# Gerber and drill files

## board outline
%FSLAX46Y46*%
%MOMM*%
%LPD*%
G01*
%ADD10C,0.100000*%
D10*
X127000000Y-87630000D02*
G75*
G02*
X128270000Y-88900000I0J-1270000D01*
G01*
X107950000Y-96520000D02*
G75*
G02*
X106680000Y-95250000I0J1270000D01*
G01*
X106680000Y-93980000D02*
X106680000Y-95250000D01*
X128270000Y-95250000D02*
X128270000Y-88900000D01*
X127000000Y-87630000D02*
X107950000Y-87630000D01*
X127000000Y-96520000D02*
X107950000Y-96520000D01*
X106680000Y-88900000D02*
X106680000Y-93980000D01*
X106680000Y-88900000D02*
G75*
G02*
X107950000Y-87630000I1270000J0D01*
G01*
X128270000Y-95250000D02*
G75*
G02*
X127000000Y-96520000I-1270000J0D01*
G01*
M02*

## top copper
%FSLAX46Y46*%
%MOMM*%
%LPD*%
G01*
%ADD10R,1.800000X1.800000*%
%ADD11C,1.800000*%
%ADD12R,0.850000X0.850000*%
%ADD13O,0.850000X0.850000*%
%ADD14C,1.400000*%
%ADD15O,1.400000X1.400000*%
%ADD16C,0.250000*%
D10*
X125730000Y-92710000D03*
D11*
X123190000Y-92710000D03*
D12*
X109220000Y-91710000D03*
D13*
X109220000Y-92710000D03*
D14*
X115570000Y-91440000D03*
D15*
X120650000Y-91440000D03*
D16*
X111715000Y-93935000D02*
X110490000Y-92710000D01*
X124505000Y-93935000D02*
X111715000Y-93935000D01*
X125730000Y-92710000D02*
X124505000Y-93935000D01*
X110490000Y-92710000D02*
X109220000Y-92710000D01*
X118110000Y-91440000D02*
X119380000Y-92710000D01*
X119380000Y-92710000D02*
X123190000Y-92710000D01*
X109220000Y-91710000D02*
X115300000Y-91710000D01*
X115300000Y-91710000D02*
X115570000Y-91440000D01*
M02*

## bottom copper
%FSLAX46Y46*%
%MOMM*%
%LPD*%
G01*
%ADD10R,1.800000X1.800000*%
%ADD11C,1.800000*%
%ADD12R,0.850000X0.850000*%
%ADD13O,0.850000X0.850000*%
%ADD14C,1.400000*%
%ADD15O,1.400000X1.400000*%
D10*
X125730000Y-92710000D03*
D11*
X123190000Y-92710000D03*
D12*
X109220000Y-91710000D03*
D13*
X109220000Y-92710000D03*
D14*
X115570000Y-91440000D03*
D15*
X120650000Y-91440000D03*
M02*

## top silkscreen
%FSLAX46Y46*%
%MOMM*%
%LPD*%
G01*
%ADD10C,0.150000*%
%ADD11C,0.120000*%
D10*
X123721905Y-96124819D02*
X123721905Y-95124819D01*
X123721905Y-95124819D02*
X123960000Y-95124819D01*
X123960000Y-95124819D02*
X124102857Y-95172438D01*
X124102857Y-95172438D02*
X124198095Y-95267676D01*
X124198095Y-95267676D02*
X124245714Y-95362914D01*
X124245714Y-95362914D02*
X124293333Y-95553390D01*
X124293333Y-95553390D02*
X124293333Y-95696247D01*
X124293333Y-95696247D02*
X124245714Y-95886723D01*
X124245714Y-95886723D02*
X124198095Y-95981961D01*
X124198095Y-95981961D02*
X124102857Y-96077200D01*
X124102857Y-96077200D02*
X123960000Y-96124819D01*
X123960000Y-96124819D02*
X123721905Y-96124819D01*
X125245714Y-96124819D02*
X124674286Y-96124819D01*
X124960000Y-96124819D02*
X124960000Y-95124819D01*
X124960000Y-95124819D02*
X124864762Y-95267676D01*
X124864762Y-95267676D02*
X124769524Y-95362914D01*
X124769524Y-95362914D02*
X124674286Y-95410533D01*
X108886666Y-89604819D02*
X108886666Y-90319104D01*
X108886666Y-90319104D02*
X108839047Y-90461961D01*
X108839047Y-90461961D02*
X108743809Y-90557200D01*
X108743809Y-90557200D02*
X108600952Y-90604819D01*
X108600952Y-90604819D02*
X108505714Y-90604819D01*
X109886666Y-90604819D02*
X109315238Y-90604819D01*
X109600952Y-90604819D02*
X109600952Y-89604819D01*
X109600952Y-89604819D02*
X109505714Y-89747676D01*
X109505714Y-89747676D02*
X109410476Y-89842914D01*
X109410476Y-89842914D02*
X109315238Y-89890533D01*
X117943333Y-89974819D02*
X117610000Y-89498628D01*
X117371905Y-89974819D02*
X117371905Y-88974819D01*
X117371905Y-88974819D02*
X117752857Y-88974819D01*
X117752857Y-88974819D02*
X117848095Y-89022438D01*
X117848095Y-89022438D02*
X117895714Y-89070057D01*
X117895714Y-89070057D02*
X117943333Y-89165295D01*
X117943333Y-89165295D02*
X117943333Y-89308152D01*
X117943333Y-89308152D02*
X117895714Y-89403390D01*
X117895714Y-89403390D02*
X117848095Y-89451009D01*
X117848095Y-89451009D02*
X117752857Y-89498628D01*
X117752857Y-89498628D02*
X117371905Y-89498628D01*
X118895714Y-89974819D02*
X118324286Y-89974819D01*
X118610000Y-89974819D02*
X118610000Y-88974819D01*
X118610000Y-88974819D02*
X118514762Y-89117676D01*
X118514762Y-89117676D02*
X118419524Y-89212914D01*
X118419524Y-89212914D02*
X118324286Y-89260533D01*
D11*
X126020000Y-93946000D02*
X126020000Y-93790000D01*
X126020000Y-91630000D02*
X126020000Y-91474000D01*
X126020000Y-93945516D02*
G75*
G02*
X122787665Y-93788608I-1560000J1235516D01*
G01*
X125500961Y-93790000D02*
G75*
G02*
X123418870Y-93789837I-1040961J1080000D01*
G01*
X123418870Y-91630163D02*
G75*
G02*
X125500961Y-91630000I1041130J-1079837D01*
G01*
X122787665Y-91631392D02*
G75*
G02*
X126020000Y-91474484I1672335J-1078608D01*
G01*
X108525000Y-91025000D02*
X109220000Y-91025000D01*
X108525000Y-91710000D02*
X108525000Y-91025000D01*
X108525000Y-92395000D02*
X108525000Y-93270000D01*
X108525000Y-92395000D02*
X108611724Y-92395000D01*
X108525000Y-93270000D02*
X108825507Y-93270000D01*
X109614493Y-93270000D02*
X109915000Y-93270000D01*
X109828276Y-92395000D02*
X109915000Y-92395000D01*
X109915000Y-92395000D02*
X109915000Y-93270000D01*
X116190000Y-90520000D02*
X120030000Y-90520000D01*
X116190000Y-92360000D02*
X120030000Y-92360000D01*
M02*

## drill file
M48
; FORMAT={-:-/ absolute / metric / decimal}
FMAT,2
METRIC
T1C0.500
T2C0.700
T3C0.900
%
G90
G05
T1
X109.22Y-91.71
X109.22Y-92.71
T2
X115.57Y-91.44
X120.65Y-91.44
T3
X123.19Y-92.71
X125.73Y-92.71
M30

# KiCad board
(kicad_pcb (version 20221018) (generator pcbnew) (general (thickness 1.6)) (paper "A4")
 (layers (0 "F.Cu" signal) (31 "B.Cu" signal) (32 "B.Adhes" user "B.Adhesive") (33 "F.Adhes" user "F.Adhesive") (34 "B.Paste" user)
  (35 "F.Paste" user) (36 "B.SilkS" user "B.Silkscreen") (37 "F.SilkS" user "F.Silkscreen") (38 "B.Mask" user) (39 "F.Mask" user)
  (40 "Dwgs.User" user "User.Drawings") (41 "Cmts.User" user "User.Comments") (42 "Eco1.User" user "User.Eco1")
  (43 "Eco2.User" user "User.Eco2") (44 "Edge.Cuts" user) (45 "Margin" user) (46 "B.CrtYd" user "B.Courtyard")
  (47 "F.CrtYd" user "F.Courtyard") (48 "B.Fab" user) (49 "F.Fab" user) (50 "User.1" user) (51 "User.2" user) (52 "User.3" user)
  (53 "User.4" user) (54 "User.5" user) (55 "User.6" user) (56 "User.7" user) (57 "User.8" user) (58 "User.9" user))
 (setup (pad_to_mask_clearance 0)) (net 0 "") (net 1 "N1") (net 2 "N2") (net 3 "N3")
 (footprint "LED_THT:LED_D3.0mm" (layer "F.Cu") (at 125.73 92.71 180)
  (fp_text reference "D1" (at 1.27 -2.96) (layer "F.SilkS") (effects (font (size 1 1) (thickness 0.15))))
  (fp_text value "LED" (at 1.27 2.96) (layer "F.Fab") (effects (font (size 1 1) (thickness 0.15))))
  (fp_line (start -0.29 -1.236) (end -0.29 -1.08) (stroke (width 0.12) (type solid)) (layer "F.SilkS"))
  (fp_line (start -0.29 1.08) (end -0.29 1.236) (stroke (width 0.12) (type solid)) (layer "F.SilkS"))
  (fp_arc (start -0.29 -1.235516) (mid 1.366487 -1.987659) (end 2.942335 -1.078608) (stroke (width 0.12) (type solid)) (layer "F.SilkS"))
  (fp_arc (start 0.229039 -1.08) (mid 1.270117 -1.5) (end 2.31113 -1.079837) (stroke (width 0.12) (type solid)) (layer "F.SilkS"))
  (fp_arc (start 2.31113 1.079837) (mid 1.270117 1.5) (end 0.229039 1.08) (stroke (width 0.12) (type solid)) (layer "F.SilkS"))
  (fp_arc (start 2.942335 1.078608) (mid 1.366487 1.987659) (end -0.29 1.235516) (stroke (width 0.12) (type solid)) (layer "F.SilkS"))
  (pad "1" thru_hole rect (at 0 0 180) (size 1.8 1.8) (drill 0.9) (layers "*.Cu" "*.Mask") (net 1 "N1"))
  (pad "2" thru_hole circle (at 2.54 0 180) (size 1.8 1.8) (drill 0.9) (layers "*.Cu" "*.Mask") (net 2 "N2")))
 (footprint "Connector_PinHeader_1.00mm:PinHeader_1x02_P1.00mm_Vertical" (layer "F.Cu") (at 109.22 91.71)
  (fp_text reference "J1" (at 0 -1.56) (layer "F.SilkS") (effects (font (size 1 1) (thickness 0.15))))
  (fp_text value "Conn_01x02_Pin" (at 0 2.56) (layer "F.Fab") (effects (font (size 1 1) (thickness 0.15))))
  (fp_line (start -0.695 -0.685) (end 0 -0.685) (stroke (width 0.12) (type solid)) (layer "F.SilkS"))
  (fp_line (start -0.695 0) (end -0.695 -0.685) (stroke (width 0.12) (type solid)) (layer "F.SilkS"))
  (fp_line (start -0.695 0.685) (end -0.695 1.56) (stroke (width 0.12) (type solid)) (layer "F.SilkS"))
  (fp_line (start -0.695 0.685) (end -0.608276 0.685) (stroke (width 0.12) (type solid)) (layer "F.SilkS"))
  (fp_line (start -0.695 1.56) (end -0.394493 1.56) (stroke (width 0.12) (type solid)) (layer "F.SilkS"))
  (fp_line (start 0.394493 1.56) (end 0.695 1.56) (stroke (width 0.12) (type solid)) (layer "F.SilkS"))
  (fp_line (start 0.608276 0.685) (end 0.695 0.685) (stroke (width 0.12) (type solid)) (layer "F.SilkS"))
  (fp_line (start 0.695 0.685) (end 0.695 1.56) (stroke (width 0.12) (type solid)) (layer "F.SilkS"))
  (pad "1" thru_hole rect (at 0 0) (size 0.85 0.85) (drill 0.5) (layers "*.Cu" "*.Mask") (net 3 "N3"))
  (pad "2" thru_hole oval (at 0 1) (size 0.85 0.85) (drill 0.5) (layers "*.Cu" "*.Mask") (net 1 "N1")))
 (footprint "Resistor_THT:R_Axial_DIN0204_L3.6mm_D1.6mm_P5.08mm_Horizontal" (layer "F.Cu") (at 115.57 91.44)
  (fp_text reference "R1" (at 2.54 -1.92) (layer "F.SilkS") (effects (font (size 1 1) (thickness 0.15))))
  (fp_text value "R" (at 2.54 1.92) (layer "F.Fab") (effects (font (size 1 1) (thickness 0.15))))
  (fp_line (start 0.62 -0.92) (end 4.46 -0.92) (stroke (width 0.12) (type solid)) (layer "F.SilkS"))
  (fp_line (start 0.62 0.92) (end 4.46 0.92) (stroke (width 0.12) (type solid)) (layer "F.SilkS"))
  (pad "1" thru_hole circle (at 0 0) (size 1.4 1.4) (drill 0.7) (layers "*.Cu" "*.Mask") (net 3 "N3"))
  (pad "2" thru_hole oval (at 5.08 0) (size 1.4 1.4) (drill 0.7) (layers "*.Cu" "*.Mask") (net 2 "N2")))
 (gr_arc (start 127 87.63) (mid 127.898026 88.001974) (end 128.27 88.9) (stroke (width 0.1) (type default)) (layer "Edge.Cuts"))
 (gr_arc (start 107.95 96.52) (mid 107.051974 96.148026) (end 106.68 95.25) (stroke (width 0.1) (type default)) (layer "Edge.Cuts"))
 (gr_line (start 106.68 93.98) (end 106.68 95.25) (stroke (width 0.1) (type default)) (layer "Edge.Cuts"))
 (gr_line (start 128.27 95.25) (end 128.27 88.9) (stroke (width 0.1) (type default)) (layer "Edge.Cuts"))
 (gr_line (start 127 87.63) (end 107.95 87.63) (stroke (width 0.1) (type default)) (layer "Edge.Cuts"))
 (gr_line (start 127 96.52) (end 107.95 96.52) (stroke (width 0.1) (type default)) (layer "Edge.Cuts"))
 (gr_line (start 106.68 88.9) (end 106.68 93.98) (stroke (width 0.1) (type default)) (layer "Edge.Cuts"))
 (gr_arc (start 106.68 88.9) (mid 107.051974 88.001974) (end 107.95 87.63) (stroke (width 0.1) (type default)) (layer "Edge.Cuts"))
 (gr_arc (start 128.27 95.25) (mid 127.898026 96.148026) (end 127 96.52) (stroke (width 0.1) (type default)) (layer "Edge.Cuts"))
 (segment (start 111.715 93.935) (end 110.49 92.71) (width 0.25) (layer "F.Cu") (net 1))
 (segment (start 124.505 93.935) (end 111.715 93.935) (width 0.25) (layer "F.Cu") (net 1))
 (segment (start 125.73 92.71) (end 124.505 93.935) (width 0.25) (layer "F.Cu") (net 1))
 (segment (start 110.49 92.71) (end 109.22 92.71) (width 0.25) (layer "F.Cu") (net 1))
 (segment (start 118.11 91.44) (end 119.38 92.71) (width 0.25) (layer "F.Cu") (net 2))
 (segment (start 119.38 92.71) (end 123.19 92.71) (width 0.25) (layer "F.Cu") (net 2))
 (segment (start 109.22 91.71) (end 115.3 91.71) (width 0.25) (layer "F.Cu") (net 3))
 (segment (start 115.3 91.71) (end 115.57 91.44) (width 0.25) (layer "F.Cu") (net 3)))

